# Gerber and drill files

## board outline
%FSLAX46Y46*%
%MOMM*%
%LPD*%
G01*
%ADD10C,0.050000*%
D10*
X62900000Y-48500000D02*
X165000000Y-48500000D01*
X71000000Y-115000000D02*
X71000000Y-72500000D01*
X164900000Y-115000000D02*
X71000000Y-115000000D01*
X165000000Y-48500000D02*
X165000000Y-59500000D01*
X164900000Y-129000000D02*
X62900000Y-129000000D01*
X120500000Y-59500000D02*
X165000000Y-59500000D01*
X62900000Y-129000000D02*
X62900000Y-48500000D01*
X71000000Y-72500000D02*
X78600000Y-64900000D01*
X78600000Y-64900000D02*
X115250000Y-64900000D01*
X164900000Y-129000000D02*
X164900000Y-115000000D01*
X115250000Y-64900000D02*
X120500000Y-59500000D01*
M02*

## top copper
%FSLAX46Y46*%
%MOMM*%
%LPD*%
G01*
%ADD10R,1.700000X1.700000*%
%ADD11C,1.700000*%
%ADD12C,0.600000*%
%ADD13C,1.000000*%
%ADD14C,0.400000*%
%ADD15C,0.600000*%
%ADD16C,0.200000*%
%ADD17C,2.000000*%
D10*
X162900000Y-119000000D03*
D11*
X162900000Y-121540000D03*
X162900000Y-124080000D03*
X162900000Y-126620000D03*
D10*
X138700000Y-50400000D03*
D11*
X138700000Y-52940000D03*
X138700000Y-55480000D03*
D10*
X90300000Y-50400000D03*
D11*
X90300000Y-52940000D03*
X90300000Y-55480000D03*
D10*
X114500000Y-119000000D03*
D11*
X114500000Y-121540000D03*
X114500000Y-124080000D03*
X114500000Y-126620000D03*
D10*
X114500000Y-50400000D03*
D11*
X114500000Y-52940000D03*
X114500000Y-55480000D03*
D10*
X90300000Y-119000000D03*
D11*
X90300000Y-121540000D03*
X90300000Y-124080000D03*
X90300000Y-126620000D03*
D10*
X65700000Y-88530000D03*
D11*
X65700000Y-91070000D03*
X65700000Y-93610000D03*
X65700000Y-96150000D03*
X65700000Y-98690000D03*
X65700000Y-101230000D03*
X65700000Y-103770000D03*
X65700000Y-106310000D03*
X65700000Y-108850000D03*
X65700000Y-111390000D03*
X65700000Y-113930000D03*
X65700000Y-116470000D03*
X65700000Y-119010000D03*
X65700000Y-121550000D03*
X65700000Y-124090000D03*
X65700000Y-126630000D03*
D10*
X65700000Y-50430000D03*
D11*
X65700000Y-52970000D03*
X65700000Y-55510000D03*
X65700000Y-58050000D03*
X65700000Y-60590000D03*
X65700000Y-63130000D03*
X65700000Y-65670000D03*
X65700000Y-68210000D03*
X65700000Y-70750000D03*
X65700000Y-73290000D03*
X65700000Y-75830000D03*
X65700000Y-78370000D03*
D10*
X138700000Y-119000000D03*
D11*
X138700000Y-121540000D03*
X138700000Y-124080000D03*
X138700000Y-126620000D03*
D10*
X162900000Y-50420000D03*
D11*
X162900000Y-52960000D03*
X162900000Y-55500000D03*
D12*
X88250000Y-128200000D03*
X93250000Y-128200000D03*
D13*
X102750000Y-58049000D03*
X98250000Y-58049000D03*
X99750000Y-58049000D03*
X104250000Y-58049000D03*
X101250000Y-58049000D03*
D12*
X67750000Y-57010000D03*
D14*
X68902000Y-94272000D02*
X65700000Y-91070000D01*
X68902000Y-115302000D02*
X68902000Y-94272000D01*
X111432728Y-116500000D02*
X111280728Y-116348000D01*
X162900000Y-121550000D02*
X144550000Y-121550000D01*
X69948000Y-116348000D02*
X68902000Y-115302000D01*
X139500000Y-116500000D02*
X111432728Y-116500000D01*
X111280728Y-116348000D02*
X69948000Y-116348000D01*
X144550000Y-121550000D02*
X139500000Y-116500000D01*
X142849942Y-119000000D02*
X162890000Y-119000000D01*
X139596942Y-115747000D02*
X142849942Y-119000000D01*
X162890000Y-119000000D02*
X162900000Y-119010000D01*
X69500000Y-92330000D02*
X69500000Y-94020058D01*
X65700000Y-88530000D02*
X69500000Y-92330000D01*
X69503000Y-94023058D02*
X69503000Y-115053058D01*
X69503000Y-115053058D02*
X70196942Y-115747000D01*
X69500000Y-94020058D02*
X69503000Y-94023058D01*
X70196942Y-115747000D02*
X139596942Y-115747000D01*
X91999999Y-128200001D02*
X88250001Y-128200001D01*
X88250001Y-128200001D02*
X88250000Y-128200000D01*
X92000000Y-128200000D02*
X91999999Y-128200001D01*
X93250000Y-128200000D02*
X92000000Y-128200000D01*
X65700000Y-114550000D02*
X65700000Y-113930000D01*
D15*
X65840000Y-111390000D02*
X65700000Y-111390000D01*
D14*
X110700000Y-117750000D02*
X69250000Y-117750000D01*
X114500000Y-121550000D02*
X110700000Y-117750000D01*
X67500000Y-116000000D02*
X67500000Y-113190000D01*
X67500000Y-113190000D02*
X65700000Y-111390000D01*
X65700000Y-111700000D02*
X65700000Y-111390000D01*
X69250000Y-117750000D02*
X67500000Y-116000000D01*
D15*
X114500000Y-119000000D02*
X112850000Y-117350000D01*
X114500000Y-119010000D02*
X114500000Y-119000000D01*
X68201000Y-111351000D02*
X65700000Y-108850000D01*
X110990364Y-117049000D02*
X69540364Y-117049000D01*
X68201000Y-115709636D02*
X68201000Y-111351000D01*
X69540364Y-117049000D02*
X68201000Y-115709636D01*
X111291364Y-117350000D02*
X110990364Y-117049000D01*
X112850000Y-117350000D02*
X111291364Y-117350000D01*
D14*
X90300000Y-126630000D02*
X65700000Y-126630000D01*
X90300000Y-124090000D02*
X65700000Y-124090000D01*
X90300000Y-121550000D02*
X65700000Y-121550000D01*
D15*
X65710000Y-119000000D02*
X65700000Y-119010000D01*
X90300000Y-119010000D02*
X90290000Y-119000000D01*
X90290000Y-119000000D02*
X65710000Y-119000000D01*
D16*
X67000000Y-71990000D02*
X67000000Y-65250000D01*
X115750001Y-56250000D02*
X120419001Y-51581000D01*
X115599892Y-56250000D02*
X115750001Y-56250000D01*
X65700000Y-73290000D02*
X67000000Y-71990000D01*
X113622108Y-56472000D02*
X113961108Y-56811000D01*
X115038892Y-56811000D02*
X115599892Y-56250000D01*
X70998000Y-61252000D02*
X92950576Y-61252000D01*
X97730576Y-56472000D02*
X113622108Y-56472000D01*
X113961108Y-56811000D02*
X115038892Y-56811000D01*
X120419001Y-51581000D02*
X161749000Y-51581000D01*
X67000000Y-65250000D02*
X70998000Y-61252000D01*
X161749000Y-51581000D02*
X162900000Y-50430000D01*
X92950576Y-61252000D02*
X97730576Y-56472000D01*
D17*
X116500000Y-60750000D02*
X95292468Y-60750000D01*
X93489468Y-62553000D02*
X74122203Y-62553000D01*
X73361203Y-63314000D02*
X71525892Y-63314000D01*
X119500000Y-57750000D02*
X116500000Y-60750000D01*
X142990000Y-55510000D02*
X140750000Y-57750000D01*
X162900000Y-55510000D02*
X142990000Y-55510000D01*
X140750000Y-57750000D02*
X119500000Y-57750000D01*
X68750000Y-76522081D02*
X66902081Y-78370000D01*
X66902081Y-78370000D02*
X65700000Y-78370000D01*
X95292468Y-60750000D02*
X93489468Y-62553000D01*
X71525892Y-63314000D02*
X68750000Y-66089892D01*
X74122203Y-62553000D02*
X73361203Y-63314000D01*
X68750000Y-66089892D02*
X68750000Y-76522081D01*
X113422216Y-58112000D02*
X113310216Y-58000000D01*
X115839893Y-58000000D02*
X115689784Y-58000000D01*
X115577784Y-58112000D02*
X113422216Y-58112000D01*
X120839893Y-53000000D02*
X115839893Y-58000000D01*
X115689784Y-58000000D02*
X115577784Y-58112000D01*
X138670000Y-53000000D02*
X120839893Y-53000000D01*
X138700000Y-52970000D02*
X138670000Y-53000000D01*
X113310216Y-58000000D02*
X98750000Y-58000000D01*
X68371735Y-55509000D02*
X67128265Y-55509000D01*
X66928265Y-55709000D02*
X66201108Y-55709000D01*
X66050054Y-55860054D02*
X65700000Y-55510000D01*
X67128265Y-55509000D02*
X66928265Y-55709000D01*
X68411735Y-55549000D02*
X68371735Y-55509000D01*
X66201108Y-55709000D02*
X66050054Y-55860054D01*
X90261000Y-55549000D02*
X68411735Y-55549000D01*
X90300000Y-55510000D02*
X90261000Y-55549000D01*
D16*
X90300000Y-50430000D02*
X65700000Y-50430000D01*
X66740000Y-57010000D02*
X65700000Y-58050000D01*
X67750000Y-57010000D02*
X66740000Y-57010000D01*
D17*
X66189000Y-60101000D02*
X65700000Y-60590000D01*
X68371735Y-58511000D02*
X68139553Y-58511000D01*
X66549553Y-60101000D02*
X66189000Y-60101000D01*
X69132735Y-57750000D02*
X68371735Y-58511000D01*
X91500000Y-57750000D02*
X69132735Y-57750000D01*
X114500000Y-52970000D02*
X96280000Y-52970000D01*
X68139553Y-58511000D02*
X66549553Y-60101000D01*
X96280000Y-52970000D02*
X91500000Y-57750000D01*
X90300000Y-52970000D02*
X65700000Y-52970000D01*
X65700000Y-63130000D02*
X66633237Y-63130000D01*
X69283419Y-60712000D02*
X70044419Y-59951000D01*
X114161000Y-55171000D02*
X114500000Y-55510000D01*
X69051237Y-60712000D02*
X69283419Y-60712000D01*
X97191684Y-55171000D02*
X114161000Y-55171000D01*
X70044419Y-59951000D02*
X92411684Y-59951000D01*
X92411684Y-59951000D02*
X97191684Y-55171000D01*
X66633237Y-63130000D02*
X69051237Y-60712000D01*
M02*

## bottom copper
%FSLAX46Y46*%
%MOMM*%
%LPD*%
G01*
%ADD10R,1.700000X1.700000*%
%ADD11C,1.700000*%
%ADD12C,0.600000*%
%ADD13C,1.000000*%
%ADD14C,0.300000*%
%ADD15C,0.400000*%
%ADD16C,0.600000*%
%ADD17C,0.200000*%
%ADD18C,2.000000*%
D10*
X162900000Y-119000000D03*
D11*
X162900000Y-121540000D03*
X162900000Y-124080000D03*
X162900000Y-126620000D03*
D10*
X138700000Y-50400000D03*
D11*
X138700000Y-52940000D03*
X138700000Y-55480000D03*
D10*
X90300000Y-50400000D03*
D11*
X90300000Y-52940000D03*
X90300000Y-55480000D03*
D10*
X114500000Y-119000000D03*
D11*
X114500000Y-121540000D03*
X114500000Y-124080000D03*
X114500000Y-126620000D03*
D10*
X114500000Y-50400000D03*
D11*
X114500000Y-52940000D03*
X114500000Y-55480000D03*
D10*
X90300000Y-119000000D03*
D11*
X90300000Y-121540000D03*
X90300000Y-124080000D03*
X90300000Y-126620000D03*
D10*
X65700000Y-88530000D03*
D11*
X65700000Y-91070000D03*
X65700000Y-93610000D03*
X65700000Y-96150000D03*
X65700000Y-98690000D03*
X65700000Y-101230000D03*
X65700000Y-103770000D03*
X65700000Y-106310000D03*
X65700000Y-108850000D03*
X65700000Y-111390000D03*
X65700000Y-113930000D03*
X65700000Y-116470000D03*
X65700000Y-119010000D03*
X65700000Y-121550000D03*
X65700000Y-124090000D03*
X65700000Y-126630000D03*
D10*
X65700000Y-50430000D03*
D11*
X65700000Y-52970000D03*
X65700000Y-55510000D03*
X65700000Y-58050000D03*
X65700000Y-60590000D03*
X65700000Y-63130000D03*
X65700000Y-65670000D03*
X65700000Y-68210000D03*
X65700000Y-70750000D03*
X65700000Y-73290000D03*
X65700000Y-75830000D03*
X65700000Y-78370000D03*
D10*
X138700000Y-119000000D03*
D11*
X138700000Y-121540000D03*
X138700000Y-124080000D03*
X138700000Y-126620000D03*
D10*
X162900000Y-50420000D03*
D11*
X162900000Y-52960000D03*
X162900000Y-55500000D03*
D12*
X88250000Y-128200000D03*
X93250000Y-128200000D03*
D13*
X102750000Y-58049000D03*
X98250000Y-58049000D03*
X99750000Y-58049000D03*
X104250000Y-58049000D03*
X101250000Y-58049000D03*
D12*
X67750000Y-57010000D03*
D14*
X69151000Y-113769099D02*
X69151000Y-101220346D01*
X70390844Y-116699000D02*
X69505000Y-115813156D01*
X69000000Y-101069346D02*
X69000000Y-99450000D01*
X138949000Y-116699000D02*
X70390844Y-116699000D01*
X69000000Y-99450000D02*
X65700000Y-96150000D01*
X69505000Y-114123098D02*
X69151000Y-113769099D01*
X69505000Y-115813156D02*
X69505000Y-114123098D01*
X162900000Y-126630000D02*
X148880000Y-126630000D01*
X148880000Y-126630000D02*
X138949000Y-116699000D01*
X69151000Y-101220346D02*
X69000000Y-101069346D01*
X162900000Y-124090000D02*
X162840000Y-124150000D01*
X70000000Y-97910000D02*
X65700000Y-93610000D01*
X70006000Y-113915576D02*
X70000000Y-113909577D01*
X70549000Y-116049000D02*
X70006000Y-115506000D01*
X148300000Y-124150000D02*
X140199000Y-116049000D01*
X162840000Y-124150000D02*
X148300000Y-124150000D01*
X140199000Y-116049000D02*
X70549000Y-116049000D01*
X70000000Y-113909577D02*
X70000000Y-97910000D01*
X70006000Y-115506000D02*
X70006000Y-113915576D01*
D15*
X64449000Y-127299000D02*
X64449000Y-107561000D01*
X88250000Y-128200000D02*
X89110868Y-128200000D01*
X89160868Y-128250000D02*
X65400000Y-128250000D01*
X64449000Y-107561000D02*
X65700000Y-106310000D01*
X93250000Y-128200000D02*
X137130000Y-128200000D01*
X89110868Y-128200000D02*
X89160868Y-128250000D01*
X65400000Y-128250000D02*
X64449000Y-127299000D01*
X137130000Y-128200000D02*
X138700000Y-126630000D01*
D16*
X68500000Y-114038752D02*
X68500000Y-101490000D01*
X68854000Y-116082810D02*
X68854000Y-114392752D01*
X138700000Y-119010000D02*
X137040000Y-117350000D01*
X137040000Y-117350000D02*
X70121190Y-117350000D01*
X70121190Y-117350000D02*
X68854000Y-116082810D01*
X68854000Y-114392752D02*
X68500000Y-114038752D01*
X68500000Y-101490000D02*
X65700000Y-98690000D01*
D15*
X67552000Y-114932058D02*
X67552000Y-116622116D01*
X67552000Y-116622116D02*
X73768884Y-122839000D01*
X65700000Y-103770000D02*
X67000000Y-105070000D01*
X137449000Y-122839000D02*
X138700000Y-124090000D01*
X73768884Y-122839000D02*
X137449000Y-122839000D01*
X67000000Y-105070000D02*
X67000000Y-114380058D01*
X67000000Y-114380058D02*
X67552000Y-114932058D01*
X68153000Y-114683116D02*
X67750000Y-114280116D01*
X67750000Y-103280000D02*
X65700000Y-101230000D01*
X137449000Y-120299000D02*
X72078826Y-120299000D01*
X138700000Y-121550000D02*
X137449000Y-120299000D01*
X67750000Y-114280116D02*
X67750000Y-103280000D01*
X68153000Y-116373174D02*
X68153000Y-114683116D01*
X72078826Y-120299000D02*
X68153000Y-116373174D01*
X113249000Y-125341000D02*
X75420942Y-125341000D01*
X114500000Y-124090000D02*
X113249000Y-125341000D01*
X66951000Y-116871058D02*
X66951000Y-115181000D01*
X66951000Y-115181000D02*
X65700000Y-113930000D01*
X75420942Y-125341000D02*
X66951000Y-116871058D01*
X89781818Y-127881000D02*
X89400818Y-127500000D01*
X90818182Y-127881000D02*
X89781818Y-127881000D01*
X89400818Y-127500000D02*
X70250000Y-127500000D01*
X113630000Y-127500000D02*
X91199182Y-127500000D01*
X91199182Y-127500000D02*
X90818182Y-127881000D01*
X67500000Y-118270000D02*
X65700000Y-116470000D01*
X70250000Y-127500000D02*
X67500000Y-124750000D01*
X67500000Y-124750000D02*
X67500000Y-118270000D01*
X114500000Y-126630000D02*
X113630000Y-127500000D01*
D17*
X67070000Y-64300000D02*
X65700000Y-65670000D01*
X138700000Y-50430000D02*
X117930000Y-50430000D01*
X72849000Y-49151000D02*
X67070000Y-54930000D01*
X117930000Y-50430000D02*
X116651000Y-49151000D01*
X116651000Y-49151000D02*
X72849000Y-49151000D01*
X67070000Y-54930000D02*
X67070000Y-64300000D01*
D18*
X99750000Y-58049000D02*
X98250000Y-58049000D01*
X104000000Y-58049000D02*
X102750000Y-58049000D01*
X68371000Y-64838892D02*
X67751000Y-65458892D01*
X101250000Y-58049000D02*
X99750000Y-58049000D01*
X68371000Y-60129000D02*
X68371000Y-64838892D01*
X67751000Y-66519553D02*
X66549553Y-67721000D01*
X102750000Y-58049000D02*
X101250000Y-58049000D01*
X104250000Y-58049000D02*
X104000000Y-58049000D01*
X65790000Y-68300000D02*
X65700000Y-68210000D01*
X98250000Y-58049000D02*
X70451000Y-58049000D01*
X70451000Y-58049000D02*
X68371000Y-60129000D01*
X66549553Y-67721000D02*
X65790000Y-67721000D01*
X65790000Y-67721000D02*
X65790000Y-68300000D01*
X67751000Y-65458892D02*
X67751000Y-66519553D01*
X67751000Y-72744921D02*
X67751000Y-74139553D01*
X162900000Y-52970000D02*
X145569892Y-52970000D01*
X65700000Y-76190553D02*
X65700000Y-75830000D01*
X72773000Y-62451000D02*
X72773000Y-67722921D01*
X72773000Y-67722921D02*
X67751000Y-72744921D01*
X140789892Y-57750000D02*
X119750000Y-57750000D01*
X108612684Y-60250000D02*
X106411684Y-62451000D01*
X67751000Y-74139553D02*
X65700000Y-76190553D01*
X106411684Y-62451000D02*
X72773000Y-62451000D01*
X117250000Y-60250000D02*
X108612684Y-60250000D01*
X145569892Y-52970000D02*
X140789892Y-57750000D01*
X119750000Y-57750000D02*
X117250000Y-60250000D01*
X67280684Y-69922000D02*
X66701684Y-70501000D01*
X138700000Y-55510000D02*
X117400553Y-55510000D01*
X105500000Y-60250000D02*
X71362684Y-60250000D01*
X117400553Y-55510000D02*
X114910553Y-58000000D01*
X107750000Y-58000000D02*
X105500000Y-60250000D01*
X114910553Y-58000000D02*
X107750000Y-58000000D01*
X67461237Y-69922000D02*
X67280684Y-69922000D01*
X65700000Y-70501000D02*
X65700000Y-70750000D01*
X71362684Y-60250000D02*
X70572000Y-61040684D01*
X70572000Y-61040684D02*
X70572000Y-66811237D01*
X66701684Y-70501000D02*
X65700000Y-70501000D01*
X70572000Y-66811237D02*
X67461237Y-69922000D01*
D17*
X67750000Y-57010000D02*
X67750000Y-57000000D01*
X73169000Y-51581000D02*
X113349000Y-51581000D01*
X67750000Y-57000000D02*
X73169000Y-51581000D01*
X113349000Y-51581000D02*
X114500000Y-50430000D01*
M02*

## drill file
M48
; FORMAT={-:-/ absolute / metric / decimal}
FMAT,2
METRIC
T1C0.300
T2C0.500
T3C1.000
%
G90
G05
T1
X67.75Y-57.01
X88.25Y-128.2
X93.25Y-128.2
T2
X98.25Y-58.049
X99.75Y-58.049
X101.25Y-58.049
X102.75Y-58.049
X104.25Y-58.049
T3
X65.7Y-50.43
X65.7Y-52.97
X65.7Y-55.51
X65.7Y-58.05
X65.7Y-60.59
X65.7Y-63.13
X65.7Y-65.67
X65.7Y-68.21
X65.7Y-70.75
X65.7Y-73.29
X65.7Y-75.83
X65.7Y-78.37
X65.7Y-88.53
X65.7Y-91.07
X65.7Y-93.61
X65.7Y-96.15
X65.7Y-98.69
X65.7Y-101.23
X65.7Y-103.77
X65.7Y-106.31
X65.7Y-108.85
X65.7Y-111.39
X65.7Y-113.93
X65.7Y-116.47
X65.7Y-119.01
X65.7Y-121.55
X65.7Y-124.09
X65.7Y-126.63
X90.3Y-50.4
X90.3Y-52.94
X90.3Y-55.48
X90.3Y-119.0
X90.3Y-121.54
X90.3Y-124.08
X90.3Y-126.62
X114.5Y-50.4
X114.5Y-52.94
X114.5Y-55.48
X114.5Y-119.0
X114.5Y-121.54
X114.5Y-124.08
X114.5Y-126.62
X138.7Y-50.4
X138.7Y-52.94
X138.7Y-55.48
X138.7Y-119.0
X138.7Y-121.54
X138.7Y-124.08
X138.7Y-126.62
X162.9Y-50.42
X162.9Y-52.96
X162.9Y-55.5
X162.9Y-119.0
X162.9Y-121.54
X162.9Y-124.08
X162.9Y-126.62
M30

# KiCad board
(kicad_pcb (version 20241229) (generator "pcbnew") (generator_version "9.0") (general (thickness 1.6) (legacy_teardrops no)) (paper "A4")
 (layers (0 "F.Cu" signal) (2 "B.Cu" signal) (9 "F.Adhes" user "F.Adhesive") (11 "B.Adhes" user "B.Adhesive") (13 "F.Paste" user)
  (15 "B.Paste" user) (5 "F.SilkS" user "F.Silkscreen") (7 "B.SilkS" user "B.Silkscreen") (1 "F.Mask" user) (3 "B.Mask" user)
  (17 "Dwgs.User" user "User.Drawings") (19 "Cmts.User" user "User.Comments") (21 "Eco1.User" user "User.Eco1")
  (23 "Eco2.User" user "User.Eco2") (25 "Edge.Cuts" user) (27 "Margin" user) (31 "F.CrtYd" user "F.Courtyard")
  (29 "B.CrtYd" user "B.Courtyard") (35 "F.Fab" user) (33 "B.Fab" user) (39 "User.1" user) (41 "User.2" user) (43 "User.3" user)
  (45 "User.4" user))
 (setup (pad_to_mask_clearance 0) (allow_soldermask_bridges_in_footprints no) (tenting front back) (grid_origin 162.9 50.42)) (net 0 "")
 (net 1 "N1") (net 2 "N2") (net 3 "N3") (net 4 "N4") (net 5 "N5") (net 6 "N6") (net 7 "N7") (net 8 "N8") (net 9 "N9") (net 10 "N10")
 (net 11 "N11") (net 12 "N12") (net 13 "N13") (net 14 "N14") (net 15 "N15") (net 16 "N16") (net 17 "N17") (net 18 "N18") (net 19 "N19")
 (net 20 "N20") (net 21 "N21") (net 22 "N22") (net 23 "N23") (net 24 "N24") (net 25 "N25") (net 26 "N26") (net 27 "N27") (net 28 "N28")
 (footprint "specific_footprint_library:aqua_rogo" (layer "F.Cu") (at 72 64 -90)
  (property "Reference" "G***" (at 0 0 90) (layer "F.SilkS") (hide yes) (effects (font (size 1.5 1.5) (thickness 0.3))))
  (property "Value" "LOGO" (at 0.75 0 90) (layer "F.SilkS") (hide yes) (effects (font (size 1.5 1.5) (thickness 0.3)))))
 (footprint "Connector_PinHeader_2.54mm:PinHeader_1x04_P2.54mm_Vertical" (layer "B.Cu") (at 162.9 119 180)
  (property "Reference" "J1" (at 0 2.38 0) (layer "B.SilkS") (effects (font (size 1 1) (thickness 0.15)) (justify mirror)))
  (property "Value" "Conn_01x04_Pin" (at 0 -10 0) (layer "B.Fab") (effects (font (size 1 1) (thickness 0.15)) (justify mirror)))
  (pad "1" thru_hole rect (at 0 0 180) (size 1.7 1.7) (drill 1) (layers "*.Cu" "*.Mask") (remove_unused_layers no) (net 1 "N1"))
  (pad "2" thru_hole circle (at 0 -2.54 180) (size 1.7 1.7) (drill 1) (layers "*.Cu" "*.Mask") (remove_unused_layers no) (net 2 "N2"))
  (pad "3" thru_hole circle (at 0 -5.08 180) (size 1.7 1.7) (drill 1) (layers "*.Cu" "*.Mask") (remove_unused_layers no) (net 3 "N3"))
  (pad "4" thru_hole circle (at 0 -7.62 180) (size 1.7 1.7) (drill 1) (layers "*.Cu" "*.Mask") (remove_unused_layers no) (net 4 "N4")))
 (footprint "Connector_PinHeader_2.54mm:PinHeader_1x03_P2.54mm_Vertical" (layer "B.Cu") (at 138.7 50.4 180)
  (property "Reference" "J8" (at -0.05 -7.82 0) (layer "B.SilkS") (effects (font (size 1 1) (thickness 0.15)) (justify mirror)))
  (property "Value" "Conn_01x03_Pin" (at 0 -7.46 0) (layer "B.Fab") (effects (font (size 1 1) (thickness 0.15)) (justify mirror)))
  (pad "1" thru_hole rect (at 0 0 180) (size 1.7 1.7) (drill 1) (layers "*.Cu" "*.Mask") (remove_unused_layers no) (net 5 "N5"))
  (pad "2" thru_hole circle (at 0 -2.54 180) (size 1.7 1.7) (drill 1) (layers "*.Cu" "*.Mask") (remove_unused_layers no) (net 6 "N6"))
  (pad "3" thru_hole circle (at 0 -5.08 180) (size 1.7 1.7) (drill 1) (layers "*.Cu" "*.Mask") (remove_unused_layers no) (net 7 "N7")))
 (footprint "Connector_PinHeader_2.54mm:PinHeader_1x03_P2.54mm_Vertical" (layer "B.Cu") (at 90.3 50.4 180)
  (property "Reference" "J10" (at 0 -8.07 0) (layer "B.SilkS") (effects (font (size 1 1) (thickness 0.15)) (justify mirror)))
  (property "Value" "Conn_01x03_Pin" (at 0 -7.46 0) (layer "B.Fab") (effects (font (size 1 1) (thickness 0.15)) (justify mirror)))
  (pad "1" thru_hole rect (at 0 0 180) (size 1.7 1.7) (drill 1) (layers "*.Cu" "*.Mask") (remove_unused_layers no) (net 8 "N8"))
  (pad "2" thru_hole circle (at 0 -2.54 180) (size 1.7 1.7) (drill 1) (layers "*.Cu" "*.Mask") (remove_unused_layers no) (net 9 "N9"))
  (pad "3" thru_hole circle (at 0 -5.08 180) (size 1.7 1.7) (drill 1) (layers "*.Cu" "*.Mask") (remove_unused_layers no) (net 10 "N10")))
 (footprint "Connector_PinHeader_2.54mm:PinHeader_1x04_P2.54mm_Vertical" (layer "B.Cu") (at 114.5 119 180)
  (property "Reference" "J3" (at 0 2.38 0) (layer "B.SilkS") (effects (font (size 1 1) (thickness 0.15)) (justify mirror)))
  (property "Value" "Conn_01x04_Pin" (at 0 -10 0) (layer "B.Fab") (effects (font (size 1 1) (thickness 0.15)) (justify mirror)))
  (pad "1" thru_hole rect (at 0 0 180) (size 1.7 1.7) (drill 1) (layers "*.Cu" "*.Mask") (remove_unused_layers no) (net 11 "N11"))
  (pad "2" thru_hole circle (at 0 -2.54 180) (size 1.7 1.7) (drill 1) (layers "*.Cu" "*.Mask") (remove_unused_layers no) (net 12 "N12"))
  (pad "3" thru_hole circle (at 0 -5.08 180) (size 1.7 1.7) (drill 1) (layers "*.Cu" "*.Mask") (remove_unused_layers no) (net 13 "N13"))
  (pad "4" thru_hole circle (at 0 -7.62 180) (size 1.7 1.7) (drill 1) (layers "*.Cu" "*.Mask") (remove_unused_layers no) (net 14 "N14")))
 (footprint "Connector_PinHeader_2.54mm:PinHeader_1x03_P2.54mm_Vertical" (layer "B.Cu") (at 114.5 50.4 180)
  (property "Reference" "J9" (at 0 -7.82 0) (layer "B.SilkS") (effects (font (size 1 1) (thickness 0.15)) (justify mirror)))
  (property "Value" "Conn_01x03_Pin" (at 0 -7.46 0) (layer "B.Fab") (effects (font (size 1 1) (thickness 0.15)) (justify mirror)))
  (pad "1" thru_hole rect (at 0 0 180) (size 1.7 1.7) (drill 1) (layers "*.Cu" "*.Mask") (remove_unused_layers no) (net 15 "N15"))
  (pad "2" thru_hole circle (at 0 -2.54 180) (size 1.7 1.7) (drill 1) (layers "*.Cu" "*.Mask") (remove_unused_layers no) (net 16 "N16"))
  (pad "3" thru_hole circle (at 0 -5.08 180) (size 1.7 1.7) (drill 1) (layers "*.Cu" "*.Mask") (remove_unused_layers no) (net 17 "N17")))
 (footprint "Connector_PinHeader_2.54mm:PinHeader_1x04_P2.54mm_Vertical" (layer "B.Cu") (at 90.3 119 180)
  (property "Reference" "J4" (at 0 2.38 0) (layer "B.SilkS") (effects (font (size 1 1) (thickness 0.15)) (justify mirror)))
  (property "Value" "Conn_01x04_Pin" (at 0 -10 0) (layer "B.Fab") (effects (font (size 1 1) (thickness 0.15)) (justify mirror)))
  (pad "1" thru_hole rect (at 0 0 180) (size 1.7 1.7) (drill 1) (layers "*.Cu" "*.Mask") (remove_unused_layers no) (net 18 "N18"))
  (pad "2" thru_hole circle (at 0 -2.54 180) (size 1.7 1.7) (drill 1) (layers "*.Cu" "*.Mask") (remove_unused_layers no) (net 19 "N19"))
  (pad "3" thru_hole circle (at 0 -5.08 180) (size 1.7 1.7) (drill 1) (layers "*.Cu" "*.Mask") (remove_unused_layers no) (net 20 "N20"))
  (pad "4" thru_hole circle (at 0 -7.62 180) (size 1.7 1.7) (drill 1) (layers "*.Cu" "*.Mask") (remove_unused_layers no) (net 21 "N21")))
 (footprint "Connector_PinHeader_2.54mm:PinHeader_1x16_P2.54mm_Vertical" (layer "B.Cu") (at 65.7 88.53 180)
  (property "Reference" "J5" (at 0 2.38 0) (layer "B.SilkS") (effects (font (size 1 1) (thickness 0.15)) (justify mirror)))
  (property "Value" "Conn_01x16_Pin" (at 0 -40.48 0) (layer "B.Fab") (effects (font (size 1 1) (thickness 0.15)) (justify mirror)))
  (pad "1" thru_hole rect (at 0 0 180) (size 1.7 1.7) (drill 1) (layers "*.Cu" "*.Mask") (remove_unused_layers no) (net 1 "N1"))
  (pad "2" thru_hole circle (at 0 -2.54 180) (size 1.7 1.7) (drill 1) (layers "*.Cu" "*.Mask") (remove_unused_layers no) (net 2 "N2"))
  (pad "3" thru_hole circle (at 0 -5.08 180) (size 1.7 1.7) (drill 1) (layers "*.Cu" "*.Mask") (remove_unused_layers no) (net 3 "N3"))
  (pad "4" thru_hole circle (at 0 -7.62 180) (size 1.7 1.7) (drill 1) (layers "*.Cu" "*.Mask") (remove_unused_layers no) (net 4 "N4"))
  (pad "5" thru_hole circle (at 0 -10.16 180) (size 1.7 1.7) (drill 1) (layers "*.Cu" "*.Mask") (remove_unused_layers no) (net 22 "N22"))
  (pad "6" thru_hole circle (at 0 -12.7 180) (size 1.7 1.7) (drill 1) (layers "*.Cu" "*.Mask") (remove_unused_layers no) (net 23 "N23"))
  (pad "7" thru_hole circle (at 0 -15.24 180) (size 1.7 1.7) (drill 1) (layers "*.Cu" "*.Mask") (remove_unused_layers no) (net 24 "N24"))
  (pad "8" thru_hole circle (at 0 -17.78 180) (size 1.7 1.7) (drill 1) (layers "*.Cu" "*.Mask") (remove_unused_layers no) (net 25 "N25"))
  (pad "9" thru_hole circle (at 0 -20.32 180) (size 1.7 1.7) (drill 1) (layers "*.Cu" "*.Mask") (remove_unused_layers no) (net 11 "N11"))
  (pad "10" thru_hole circle (at 0 -22.86 180) (size 1.7 1.7) (drill 1) (layers "*.Cu" "*.Mask") (remove_unused_layers no) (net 12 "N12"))
  (pad "11" thru_hole circle (at 0 -25.4 180) (size 1.7 1.7) (drill 1) (layers "*.Cu" "*.Mask") (remove_unused_layers no) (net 13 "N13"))
  (pad "12" thru_hole circle (at 0 -27.94 180) (size 1.7 1.7) (drill 1) (layers "*.Cu" "*.Mask") (remove_unused_layers no) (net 14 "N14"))
  (pad "13" thru_hole circle (at 0 -30.48 180) (size 1.7 1.7) (drill 1) (layers "*.Cu" "*.Mask") (remove_unused_layers no) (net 18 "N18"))
  (pad "14" thru_hole circle (at 0 -33.02 180) (size 1.7 1.7) (drill 1) (layers "*.Cu" "*.Mask") (remove_unused_layers no) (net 19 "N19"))
  (pad "15" thru_hole circle (at 0 -35.56 180) (size 1.7 1.7) (drill 1) (layers "*.Cu" "*.Mask") (remove_unused_layers no) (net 20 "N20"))
  (pad "16" thru_hole circle (at 0 -38.1 180) (size 1.7 1.7) (drill 1) (layers "*.Cu" "*.Mask") (remove_unused_layers no) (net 21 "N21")))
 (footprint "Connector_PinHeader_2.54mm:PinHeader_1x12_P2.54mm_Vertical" (layer "B.Cu") (at 65.7 50.43 180)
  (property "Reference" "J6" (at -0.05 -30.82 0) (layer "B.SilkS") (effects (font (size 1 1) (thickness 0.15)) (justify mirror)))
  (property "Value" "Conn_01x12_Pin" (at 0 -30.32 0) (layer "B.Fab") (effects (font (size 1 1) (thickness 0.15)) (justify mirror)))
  (pad "1" thru_hole rect (at 0 0 180) (size 1.7 1.7) (drill 1) (layers "*.Cu" "*.Mask") (remove_unused_layers no) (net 8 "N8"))
  (pad "2" thru_hole circle (at 0 -2.54 180) (size 1.7 1.7) (drill 1) (layers "*.Cu" "*.Mask") (remove_unused_layers no) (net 9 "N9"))
  (pad "3" thru_hole circle (at 0 -5.08 180) (size 1.7 1.7) (drill 1) (layers "*.Cu" "*.Mask") (remove_unused_layers no) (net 10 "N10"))
  (pad "4" thru_hole circle (at 0 -7.62 180) (size 1.7 1.7) (drill 1) (layers "*.Cu" "*.Mask") (remove_unused_layers no) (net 15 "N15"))
  (pad "5" thru_hole circle (at 0 -10.16 180) (size 1.7 1.7) (drill 1) (layers "*.Cu" "*.Mask") (remove_unused_layers no) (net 16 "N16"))
  (pad "6" thru_hole circle (at 0 -12.7 180) (size 1.7 1.7) (drill 1) (layers "*.Cu" "*.Mask") (remove_unused_layers no) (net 17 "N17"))
  (pad "7" thru_hole circle (at 0 -15.24 180) (size 1.7 1.7) (drill 1) (layers "*.Cu" "*.Mask") (remove_unused_layers no) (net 5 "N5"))
  (pad "8" thru_hole circle (at 0 -17.78 180) (size 1.7 1.7) (drill 1) (layers "*.Cu" "*.Mask") (remove_unused_layers no) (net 6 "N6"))
  (pad "9" thru_hole circle (at 0 -20.32 180) (size 1.7 1.7) (drill 1) (layers "*.Cu" "*.Mask") (remove_unused_layers no) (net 7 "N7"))
  (pad "10" thru_hole circle (at 0 -22.86 180) (size 1.7 1.7) (drill 1) (layers "*.Cu" "*.Mask") (remove_unused_layers no) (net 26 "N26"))
  (pad "11" thru_hole circle (at 0 -25.4 180) (size 1.7 1.7) (drill 1) (layers "*.Cu" "*.Mask") (remove_unused_layers no) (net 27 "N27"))
  (pad "12" thru_hole circle (at 0 -27.94 180) (size 1.7 1.7) (drill 1) (layers "*.Cu" "*.Mask") (remove_unused_layers no) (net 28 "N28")))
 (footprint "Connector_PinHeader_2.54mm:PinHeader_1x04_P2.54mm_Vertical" (layer "B.Cu") (at 138.7 119 180)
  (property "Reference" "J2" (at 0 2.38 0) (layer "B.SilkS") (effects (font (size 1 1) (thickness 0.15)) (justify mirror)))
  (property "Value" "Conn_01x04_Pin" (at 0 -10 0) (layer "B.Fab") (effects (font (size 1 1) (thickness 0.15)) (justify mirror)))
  (pad "1" thru_hole rect (at 0 0 180) (size 1.7 1.7) (drill 1) (layers "*.Cu" "*.Mask") (remove_unused_layers no) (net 22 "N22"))
  (pad "2" thru_hole circle (at 0 -2.54 180) (size 1.7 1.7) (drill 1) (layers "*.Cu" "*.Mask") (remove_unused_layers no) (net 23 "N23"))
  (pad "3" thru_hole circle (at 0 -5.08 180) (size 1.7 1.7) (drill 1) (layers "*.Cu" "*.Mask") (remove_unused_layers no) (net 24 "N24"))
  (pad "4" thru_hole circle (at 0 -7.62 180) (size 1.7 1.7) (drill 1) (layers "*.Cu" "*.Mask") (remove_unused_layers no) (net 25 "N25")))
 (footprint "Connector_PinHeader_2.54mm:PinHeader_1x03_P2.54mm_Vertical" (layer "B.Cu") (at 162.9 50.42 180)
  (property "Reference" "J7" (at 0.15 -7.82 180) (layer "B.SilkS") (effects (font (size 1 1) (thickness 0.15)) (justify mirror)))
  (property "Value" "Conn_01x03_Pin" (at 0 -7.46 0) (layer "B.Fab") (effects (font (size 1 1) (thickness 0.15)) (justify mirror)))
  (pad "1" thru_hole rect (at 0 0 180) (size 1.7 1.7) (drill 1) (layers "*.Cu" "*.Mask") (remove_unused_layers no) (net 26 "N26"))
  (pad "2" thru_hole circle (at 0 -2.54 180) (size 1.7 1.7) (drill 1) (layers "*.Cu" "*.Mask") (remove_unused_layers no) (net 27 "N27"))
  (pad "3" thru_hole circle (at 0 -5.08 180) (size 1.7 1.7) (drill 1) (layers "*.Cu" "*.Mask") (remove_unused_layers no) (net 28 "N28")))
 (gr_line (start 62.9 48.5) (end 165 48.5) (stroke (width 0.05) (type default)) (layer "Edge.Cuts"))
 (gr_line (start 71 115) (end 71 72.5) (stroke (width 0.05) (type default)) (layer "Edge.Cuts"))
 (gr_line (start 164.9 115) (end 71 115) (stroke (width 0.05) (type default)) (layer "Edge.Cuts"))
 (gr_line (start 165 48.5) (end 165 59.5) (stroke (width 0.05) (type default)) (layer "Edge.Cuts"))
 (gr_line (start 164.9 129) (end 62.9 129) (stroke (width 0.05) (type solid)) (layer "Edge.Cuts"))
 (gr_line (start 120.5 59.5) (end 165 59.5) (stroke (width 0.05) (type default)) (layer "Edge.Cuts"))
 (gr_line (start 62.9 129) (end 62.9 48.5) (stroke (width 0.05) (type default)) (layer "Edge.Cuts"))
 (gr_line (start 71 72.5) (end 78.6 64.9) (stroke (width 0.05) (type default)) (layer "Edge.Cuts"))
 (gr_line (start 78.6 64.9) (end 115.25 64.9) (stroke (width 0.05) (type default)) (layer "Edge.Cuts"))
 (gr_line (start 164.9 129) (end 164.9 115) (stroke (width 0.05) (type default)) (layer "Edge.Cuts"))
 (gr_line (start 115.25 64.9) (end 120.5 59.5) (stroke (width 0.05) (type default)) (layer "Edge.Cuts"))
 (segment (start 68.902 94.272) (end 65.7 91.07) (width 0.4) (layer "F.Cu") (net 2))
 (segment (start 68.902 115.302) (end 68.902 94.272) (width 0.4) (layer "F.Cu") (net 2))
 (segment (start 111.432728 116.5) (end 111.280728 116.348) (width 0.4) (layer "F.Cu") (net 2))
 (segment (start 162.9 121.55) (end 144.55 121.55) (width 0.4) (layer "F.Cu") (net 2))
 (segment (start 69.948 116.348) (end 68.902 115.302) (width 0.4) (layer "F.Cu") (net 2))
 (segment (start 139.5 116.5) (end 111.432728 116.5) (width 0.4) (layer "F.Cu") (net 2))
 (segment (start 111.280728 116.348) (end 69.948 116.348) (width 0.4) (layer "F.Cu") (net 2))
 (segment (start 144.55 121.55) (end 139.5 116.5) (width 0.4) (layer "F.Cu") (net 2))
 (segment (start 69.151 113.769099) (end 69.151 101.220346) (width 0.3) (layer "B.Cu") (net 4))
 (segment (start 70.390844 116.699) (end 69.505 115.813156) (width 0.3) (layer "B.Cu") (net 4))
 (segment (start 69 101.069346) (end 69 99.45) (width 0.3) (layer "B.Cu") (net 4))
 (segment (start 138.949 116.699) (end 70.390844 116.699) (width 0.3) (layer "B.Cu") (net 4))
 (segment (start 69 99.45) (end 65.7 96.15) (width 0.3) (layer "B.Cu") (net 4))
 (segment (start 69.505 114.123098) (end 69.151 113.769099) (width 0.3) (layer "B.Cu") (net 4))
 (segment (start 69.505 115.813156) (end 69.505 114.123098) (width 0.3) (layer "B.Cu") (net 4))
 (segment (start 162.9 126.63) (end 148.88 126.63) (width 0.3) (layer "B.Cu") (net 4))
 (segment (start 148.88 126.63) (end 138.949 116.699) (width 0.3) (layer "B.Cu") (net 4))
 (segment (start 69.151 101.220346) (end 69 101.069346) (width 0.3) (layer "B.Cu") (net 4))
 (segment (start 142.849942 119) (end 162.89 119) (width 0.4) (layer "F.Cu") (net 1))
 (segment (start 139.596942 115.747) (end 142.849942 119) (width 0.4) (layer "F.Cu") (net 1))
 (segment (start 162.89 119) (end 162.9 119.01) (width 0.4) (layer "F.Cu") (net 1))
 (segment (start 69.5 92.33) (end 69.5 94.020058) (width 0.4) (layer "F.Cu") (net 1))
 (segment (start 65.7 88.53) (end 69.5 92.33) (width 0.4) (layer "F.Cu") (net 1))
 (segment (start 69.503 94.023058) (end 69.503 115.053058) (width 0.4) (layer "F.Cu") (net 1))
 (segment (start 69.503 115.053058) (end 70.196942 115.747) (width 0.4) (layer "F.Cu") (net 1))
 (segment (start 69.5 94.020058) (end 69.503 94.023058) (width 0.4) (layer "F.Cu") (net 1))
 (segment (start 70.196942 115.747) (end 139.596942 115.747) (width 0.4) (layer "F.Cu") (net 1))
 (segment (start 162.9 124.09) (end 162.84 124.15) (width 0.3) (layer "B.Cu") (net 3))
 (segment (start 70 97.91) (end 65.7 93.61) (width 0.3) (layer "B.Cu") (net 3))
 (segment (start 70.006 113.915576) (end 70 113.909577) (width 0.3) (layer "B.Cu") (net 3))
 (segment (start 70.549 116.049) (end 70.006 115.506) (width 0.3) (layer "B.Cu") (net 3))
 (segment (start 148.3 124.15) (end 140.199 116.049) (width 0.3) (layer "B.Cu") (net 3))
 (segment (start 162.84 124.15) (end 148.3 124.15) (width 0.3) (layer "B.Cu") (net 3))
 (segment (start 140.199 116.049) (end 70.549 116.049) (width 0.3) (layer "B.Cu") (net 3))
 (segment (start 70 113.909577) (end 70 97.91) (width 0.3) (layer "B.Cu") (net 3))
 (segment (start 70.006 115.506) (end 70.006 113.915576) (width 0.3) (layer "B.Cu") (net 3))
 (segment (start 91.999999 128.200001) (end 88.250001 128.200001) (width 0.4) (layer "F.Cu") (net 25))
 (segment (start 88.250001 128.200001) (end 88.25 128.2) (width 0.4) (layer "F.Cu") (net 25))
 (segment (start 92 128.2) (end 91.999999 128.200001) (width 0.4) (layer "F.Cu") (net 25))
 (segment (start 93.25 128.2) (end 92 128.2) (width 0.4) (layer "F.Cu") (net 25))
 (via (at 88.25 128.2) (size 0.6) (drill 0.3) (layers "F.Cu" "B.Cu") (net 25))
 (via (at 93.25 128.2) (size 0.6) (drill 0.3) (layers "F.Cu" "B.Cu") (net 25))
 (segment (start 64.449 127.299) (end 64.449 107.561) (width 0.4) (layer "B.Cu") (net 25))
 (segment (start 88.25 128.2) (end 89.110868 128.2) (width 0.4) (layer "B.Cu") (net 25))
 (segment (start 89.160868 128.25) (end 65.4 128.25) (width 0.4) (layer "B.Cu") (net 25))
 (segment (start 64.449 107.561) (end 65.7 106.31) (width 0.4) (layer "B.Cu") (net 25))
 (segment (start 93.25 128.2) (end 137.13 128.2) (width 0.4) (layer "B.Cu") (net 25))
 (segment (start 89.110868 128.2) (end 89.160868 128.25) (width 0.4) (layer "B.Cu") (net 25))
 (segment (start 65.4 128.25) (end 64.449 127.299) (width 0.4) (layer "B.Cu") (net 25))
 (segment (start 137.13 128.2) (end 138.7 126.63) (width 0.4) (layer "B.Cu") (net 25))
 (segment (start 68.5 114.038752) (end 68.5 101.49) (width 0.6) (layer "B.Cu") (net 22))
 (segment (start 68.854 116.08281) (end 68.854 114.392752) (width 0.6) (layer "B.Cu") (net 22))
 (segment (start 138.7 119.01) (end 137.04 117.35) (width 0.6) (layer "B.Cu") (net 22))
 (segment (start 137.04 117.35) (end 70.12119 117.35) (width 0.6) (layer "B.Cu") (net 22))
 (segment (start 70.12119 117.35) (end 68.854 116.08281) (width 0.6) (layer "B.Cu") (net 22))
 (segment (start 68.854 114.392752) (end 68.5 114.038752) (width 0.6) (layer "B.Cu") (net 22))
 (segment (start 68.5 101.49) (end 65.7 98.69) (width 0.6) (layer "B.Cu") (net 22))
 (segment (start 67.552 114.932058) (end 67.552 116.622116) (width 0.4) (layer "B.Cu") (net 24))
 (segment (start 67.552 116.622116) (end 73.768884 122.839) (width 0.4) (layer "B.Cu") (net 24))
 (segment (start 65.7 103.77) (end 67 105.07) (width 0.4) (layer "B.Cu") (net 24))
 (segment (start 137.449 122.839) (end 138.7 124.09) (width 0.4) (layer "B.Cu") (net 24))
 (segment (start 73.768884 122.839) (end 137.449 122.839) (width 0.4) (layer "B.Cu") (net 24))
 (segment (start 67 105.07) (end 67 114.380058) (width 0.4) (layer "B.Cu") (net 24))
 (segment (start 67 114.380058) (end 67.552 114.932058) (width 0.4) (layer "B.Cu") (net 24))
 (segment (start 68.153 114.683116) (end 67.75 114.280116) (width 0.4) (layer "B.Cu") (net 23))
 (segment (start 67.75 103.28) (end 65.7 101.23) (width 0.4) (layer "B.Cu") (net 23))
 (segment (start 137.449 120.299) (end 72.078826 120.299) (width 0.4) (layer "B.Cu") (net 23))
 (segment (start 138.7 121.55) (end 137.449 120.299) (width 0.4) (layer "B.Cu") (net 23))
 (segment (start 67.75 114.280116) (end 67.75 103.28) (width 0.4) (layer "B.Cu") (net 23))
 (segment (start 68.153 116.373174) (end 68.153 114.683116) (width 0.4) (layer "B.Cu") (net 23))
 (segment (start 72.078826 120.299) (end 68.153 116.373174) (width 0.4) (layer "B.Cu") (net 23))
 (segment (start 65.7 114.55) (end 65.7 113.93) (width 0.4) (layer "F.Cu") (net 13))
 (segment (start 113.249 125.341) (end 75.420942 125.341) (width 0.4) (layer "B.Cu") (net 13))
 (segment (start 114.5 124.09) (end 113.249 125.341) (width 0.4) (layer "B.Cu") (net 13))
 (segment (start 66.951 116.871058) (end 66.951 115.181) (width 0.4) (layer "B.Cu") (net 13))
 (segment (start 66.951 115.181) (end 65.7 113.93) (width 0.4) (layer "B.Cu") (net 13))
 (segment (start 75.420942 125.341) (end 66.951 116.871058) (width 0.4) (layer "B.Cu") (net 13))
 (segment (start 65.84 111.39) (end 65.7 111.39) (width 0.6) (layer "F.Cu") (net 12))
 (segment (start 110.7 117.75) (end 69.25 117.75) (width 0.4) (layer "F.Cu") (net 12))
 (segment (start 114.5 121.55) (end 110.7 117.75) (width 0.4) (layer "F.Cu") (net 12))
 (segment (start 67.5 116) (end 67.5 113.19) (width 0.4) (layer "F.Cu") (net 12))
 (segment (start 67.5 113.19) (end 65.7 111.39) (width 0.4) (layer "F.Cu") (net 12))
 (segment (start 65.7 111.7) (end 65.7 111.39) (width 0.4) (layer "F.Cu") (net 12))
 (segment (start 69.25 117.75) (end 67.5 116) (width 0.4) (layer "F.Cu") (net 12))
 (segment (start 114.5 119) (end 112.85 117.35) (width 0.6) (layer "F.Cu") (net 11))
 (segment (start 114.5 119.01) (end 114.5 119) (width 0.6) (layer "F.Cu") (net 11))
 (segment (start 68.201 111.351) (end 65.7 108.85) (width 0.6) (layer "F.Cu") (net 11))
 (segment (start 110.990364 117.049) (end 69.540364 117.049) (width 0.6) (layer "F.Cu") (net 11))
 (segment (start 68.201 115.709636) (end 68.201 111.351) (width 0.6) (layer "F.Cu") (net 11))
 (segment (start 69.540364 117.049) (end 68.201 115.709636) (width 0.6) (layer "F.Cu") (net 11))
 (segment (start 111.291364 117.35) (end 110.990364 117.049) (width 0.6) (layer "F.Cu") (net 11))
 (segment (start 112.85 117.35) (end 111.291364 117.35) (width 0.6) (layer "F.Cu") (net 11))
 (segment (start 89.781818 127.881) (end 89.400818 127.5) (width 0.4) (layer "B.Cu") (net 14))
 (segment (start 90.818182 127.881) (end 89.781818 127.881) (width 0.4) (layer "B.Cu") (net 14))
 (segment (start 89.400818 127.5) (end 70.25 127.5) (width 0.4) (layer "B.Cu") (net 14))
 (segment (start 113.63 127.5) (end 91.199182 127.5) (width 0.4) (layer "B.Cu") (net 14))
 (segment (start 91.199182 127.5) (end 90.818182 127.881) (width 0.4) (layer "B.Cu") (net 14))
 (segment (start 67.5 118.27) (end 65.7 116.47) (width 0.4) (layer "B.Cu") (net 14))
 (segment (start 70.25 127.5) (end 67.5 124.75) (width 0.4) (layer "B.Cu") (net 14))
 (segment (start 67.5 124.75) (end 67.5 118.27) (width 0.4) (layer "B.Cu") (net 14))
 (segment (start 114.5 126.63) (end 113.63 127.5) (width 0.4) (layer "B.Cu") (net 14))
 (segment (start 90.3 126.63) (end 65.7 126.63) (width 0.4) (layer "F.Cu") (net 21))
 (segment (start 90.3 124.09) (end 65.7 124.09) (width 0.4) (layer "F.Cu") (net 20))
 (segment (start 90.3 121.55) (end 65.7 121.55) (width 0.4) (layer "F.Cu") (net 19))
 (segment (start 65.71 119) (end 65.7 119.01) (width 0.6) (layer "F.Cu") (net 18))
 (segment (start 90.3 119.01) (end 90.29 119) (width 0.6) (layer "F.Cu") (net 18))
 (segment (start 90.29 119) (end 65.71 119) (width 0.6) (layer "F.Cu") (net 18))
 (segment (start 67.07 64.3) (end 65.7 65.67) (width 0.2) (layer "B.Cu") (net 5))
 (segment (start 138.7 50.43) (end 117.93 50.43) (width 0.2) (layer "B.Cu") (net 5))
 (segment (start 72.849 49.151) (end 67.07 54.93) (width 0.2) (layer "B.Cu") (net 5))
 (segment (start 117.93 50.43) (end 116.651 49.151) (width 0.2) (layer "B.Cu") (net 5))
 (segment (start 116.651 49.151) (end 72.849 49.151) (width 0.2) (layer "B.Cu") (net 5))
 (segment (start 67.07 54.93) (end 67.07 64.3) (width 0.2) (layer "B.Cu") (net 5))
 (segment (start 67 71.99) (end 67 65.25) (width 0.2) (layer "F.Cu") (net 26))
 (segment (start 115.750001 56.25) (end 120.419001 51.581) (width 0.2) (layer "F.Cu") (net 26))
 (segment (start 115.599892 56.25) (end 115.750001 56.25) (width 0.2) (layer "F.Cu") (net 26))
 (segment (start 65.7 73.29) (end 67 71.99) (width 0.2) (layer "F.Cu") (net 26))
 (segment (start 113.622108 56.472) (end 113.961108 56.811) (width 0.2) (layer "F.Cu") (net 26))
 (segment (start 115.038892 56.811) (end 115.599892 56.25) (width 0.2) (layer "F.Cu") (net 26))
 (segment (start 70.998 61.252) (end 92.950576 61.252) (width 0.2) (layer "F.Cu") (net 26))
 (segment (start 97.730576 56.472) (end 113.622108 56.472) (width 0.2) (layer "F.Cu") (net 26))
 (segment (start 113.961108 56.811) (end 115.038892 56.811) (width 0.2) (layer "F.Cu") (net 26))
 (segment (start 120.419001 51.581) (end 161.749 51.581) (width 0.2) (layer "F.Cu") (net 26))
 (segment (start 67 65.25) (end 70.998 61.252) (width 0.2) (layer "F.Cu") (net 26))
 (segment (start 161.749 51.581) (end 162.9 50.43) (width 0.2) (layer "F.Cu") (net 26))
 (segment (start 92.950576 61.252) (end 97.730576 56.472) (width 0.2) (layer "F.Cu") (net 26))
 (segment (start 116.5 60.75) (end 95.292468 60.75) (width 2) (layer "F.Cu") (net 28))
 (segment (start 93.489468 62.553) (end 74.122203 62.553) (width 2) (layer "F.Cu") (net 28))
 (segment (start 73.361203 63.314) (end 71.525892 63.314) (width 2) (layer "F.Cu") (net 28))
 (segment (start 119.5 57.75) (end 116.5 60.75) (width 2) (layer "F.Cu") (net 28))
 (segment (start 142.99 55.51) (end 140.75 57.75) (width 2) (layer "F.Cu") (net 28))
 (segment (start 162.9 55.51) (end 142.99 55.51) (width 2) (layer "F.Cu") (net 28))
 (segment (start 140.75 57.75) (end 119.5 57.75) (width 2) (layer "F.Cu") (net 28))
 (segment (start 68.75 76.522081) (end 66.902081 78.37) (width 2) (layer "F.Cu") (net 28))
 (segment (start 66.902081 78.37) (end 65.7 78.37) (width 2) (layer "F.Cu") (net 28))
 (segment (start 95.292468 60.75) (end 93.489468 62.553) (width 2) (layer "F.Cu") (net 28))
 (segment (start 71.525892 63.314) (end 68.75 66.089892) (width 2) (layer "F.Cu") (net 28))
 (segment (start 74.122203 62.553) (end 73.361203 63.314) (width 2) (layer "F.Cu") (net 28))
 (segment (start 68.75 66.089892) (end 68.75 76.522081) (width 2) (layer "F.Cu") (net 28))
 (segment (start 113.422216 58.112) (end 113.310216 58) (width 2) (layer "F.Cu") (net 6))
 (segment (start 115.839893 58) (end 115.689784 58) (width 2) (layer "F.Cu") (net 6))
 (segment (start 115.577784 58.112) (end 113.422216 58.112) (width 2) (layer "F.Cu") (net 6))
 (segment (start 120.839893 53) (end 115.839893 58) (width 2) (layer "F.Cu") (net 6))
 (segment (start 115.689784 58) (end 115.577784 58.112) (width 2) (layer "F.Cu") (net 6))
 (segment (start 138.67 53) (end 120.839893 53) (width 2) (layer "F.Cu") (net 6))
 (segment (start 138.7 52.97) (end 138.67 53) (width 2) (layer "F.Cu") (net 6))
 (segment (start 113.310216 58) (end 98.75 58) (width 2) (layer "F.Cu") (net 6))
 (via (at 102.75 58.049) (size 1) (drill 0.5) (layers "F.Cu" "B.Cu") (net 6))
 (via (at 98.25 58.049) (size 1) (drill 0.5) (layers "F.Cu" "B.Cu") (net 6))
 (via (at 99.75 58.049) (size 1) (drill 0.5) (layers "F.Cu" "B.Cu") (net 6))
 (via (at 104.25 58.049) (size 1) (drill 0.5) (layers "F.Cu" "B.Cu") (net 6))
 (via (at 101.25 58.049) (size 1) (drill 0.5) (layers "F.Cu" "B.Cu") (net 6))
 (segment (start 99.75 58.049) (end 98.25 58.049) (width 2) (layer "B.Cu") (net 6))
 (segment (start 104 58.049) (end 102.75 58.049) (width 2) (layer "B.Cu") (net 6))
 (segment (start 68.371 64.838892) (end 67.751 65.458892) (width 2) (layer "B.Cu") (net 6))
 (segment (start 101.25 58.049) (end 99.75 58.049) (width 2) (layer "B.Cu") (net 6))
 (segment (start 68.371 60.129) (end 68.371 64.838892) (width 2) (layer "B.Cu") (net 6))
 (segment (start 67.751 66.519553) (end 66.549553 67.721) (width 2) (layer "B.Cu") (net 6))
 (segment (start 102.75 58.049) (end 101.25 58.049) (width 2) (layer "B.Cu") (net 6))
 (segment (start 104.25 58.049) (end 104 58.049) (width 2) (layer "B.Cu") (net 6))
 (segment (start 65.79 68.3) (end 65.7 68.21) (width 2) (layer "B.Cu") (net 6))
 (segment (start 98.25 58.049) (end 70.451 58.049) (width 2) (layer "B.Cu") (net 6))
 (segment (start 70.451 58.049) (end 68.371 60.129) (width 2) (layer "B.Cu") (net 6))
 (segment (start 66.549553 67.721) (end 65.79 67.721) (width 2) (layer "B.Cu") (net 6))
 (segment (start 65.79 67.721) (end 65.79 68.3) (width 2) (layer "B.Cu") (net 6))
 (segment (start 67.751 65.458892) (end 67.751 66.519553) (width 2) (layer "B.Cu") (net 6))
 (segment (start 67.751 72.744921) (end 67.751 74.139553) (width 2) (layer "B.Cu") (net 27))
 (segment (start 162.9 52.97) (end 145.569892 52.97) (width 2) (layer "B.Cu") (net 27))
 (segment (start 65.7 76.190553) (end 65.7 75.83) (width 2) (layer "B.Cu") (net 27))
 (segment (start 72.773 62.451) (end 72.773 67.722921) (width 2) (layer "B.Cu") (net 27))
 (segment (start 72.773 67.722921) (end 67.751 72.744921) (width 2) (layer "B.Cu") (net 27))
 (segment (start 140.789892 57.75) (end 119.75 57.75) (width 2) (layer "B.Cu") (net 27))
 (segment (start 108.612684 60.25) (end 106.411684 62.451) (width 2) (layer "B.Cu") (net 27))
 (segment (start 67.751 74.139553) (end 65.7 76.190553) (width 2) (layer "B.Cu") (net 27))
 (segment (start 106.411684 62.451) (end 72.773 62.451) (width 2) (layer "B.Cu") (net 27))
 (segment (start 117.25 60.25) (end 108.612684 60.25) (width 2) (layer "B.Cu") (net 27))
 (segment (start 145.569892 52.97) (end 140.789892 57.75) (width 2) (layer "B.Cu") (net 27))
 (segment (start 119.75 57.75) (end 117.25 60.25) (width 2) (layer "B.Cu") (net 27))
 (segment (start 67.280684 69.922) (end 66.701684 70.501) (width 2) (layer "B.Cu") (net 7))
 (segment (start 138.7 55.51) (end 117.400553 55.51) (width 2) (layer "B.Cu") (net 7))
 (segment (start 105.5 60.25) (end 71.362684 60.25) (width 2) (layer "B.Cu") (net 7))
 (segment (start 117.400553 55.51) (end 114.910553 58) (width 2) (layer "B.Cu") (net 7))
 (segment (start 107.75 58) (end 105.5 60.25) (width 2) (layer "B.Cu") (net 7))
 (segment (start 114.910553 58) (end 107.75 58) (width 2) (layer "B.Cu") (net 7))
 (segment (start 67.461237 69.922) (end 67.280684 69.922) (width 2) (layer "B.Cu") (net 7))
 (segment (start 65.7 70.501) (end 65.7 70.75) (width 2) (layer "B.Cu") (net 7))
 (segment (start 71.362684 60.25) (end 70.572 61.040684) (width 2) (layer "B.Cu") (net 7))
 (segment (start 70.572 61.040684) (end 70.572 66.811237) (width 2) (layer "B.Cu") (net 7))
 (segment (start 66.701684 70.501) (end 65.7 70.501) (width 2) (layer "B.Cu") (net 7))
 (segment (start 70.572 66.811237) (end 67.461237 69.922) (width 2) (layer "B.Cu") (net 7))
 (segment (start 68.371735 55.509) (end 67.128265 55.509) (width 2) (layer "F.Cu") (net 10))
 (segment (start 66.928265 55.709) (end 66.201108 55.709) (width 2) (layer "F.Cu") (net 10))
 (segment (start 66.050054 55.860054) (end 65.7 55.51) (width 2) (layer "F.Cu") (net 10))
 (segment (start 67.128265 55.509) (end 66.928265 55.709) (width 2) (layer "F.Cu") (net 10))
 (segment (start 68.411735 55.549) (end 68.371735 55.509) (width 2) (layer "F.Cu") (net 10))
 (segment (start 66.201108 55.709) (end 66.050054 55.860054) (width 2) (layer "F.Cu") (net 10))
 (segment (start 90.261 55.549) (end 68.411735 55.549) (width 2) (layer "F.Cu") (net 10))
 (segment (start 90.3 55.51) (end 90.261 55.549) (width 2) (layer "F.Cu") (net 10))
 (segment (start 90.3 50.43) (end 65.7 50.43) (width 0.2) (layer "F.Cu") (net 8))
 (segment (start 66.74 57.01) (end 65.7 58.05) (width 0.2) (layer "F.Cu") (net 15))
 (segment (start 67.75 57.01) (end 66.74 57.01) (width 0.2) (layer "F.Cu") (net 15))
 (via (at 67.75 57.01) (size 0.6) (drill 0.3) (layers "F.Cu" "B.Cu") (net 15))
 (segment (start 67.75 57.01) (end 67.75 57) (width 0.2) (layer "B.Cu") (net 15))
 (segment (start 73.169 51.581) (end 113.349 51.581) (width 0.2) (layer "B.Cu") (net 15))
 (segment (start 67.75 57) (end 73.169 51.581) (width 0.2) (layer "B.Cu") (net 15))
 (segment (start 113.349 51.581) (end 114.5 50.43) (width 0.2) (layer "B.Cu") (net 15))
 (segment (start 66.189 60.101) (end 65.7 60.59) (width 2) (layer "F.Cu") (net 16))
 (segment (start 68.371735 58.511) (end 68.139553 58.511) (width 2) (layer "F.Cu") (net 16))
 (segment (start 66.549553 60.101) (end 66.189 60.101) (width 2) (layer "F.Cu") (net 16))
 (segment (start 69.132735 57.75) (end 68.371735 58.511) (width 2) (layer "F.Cu") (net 16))
 (segment (start 91.5 57.75) (end 69.132735 57.75) (width 2) (layer "F.Cu") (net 16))
 (segment (start 114.5 52.97) (end 96.28 52.97) (width 2) (layer "F.Cu") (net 16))
 (segment (start 68.139553 58.511) (end 66.549553 60.101) (width 2) (layer "F.Cu") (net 16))
 (segment (start 96.28 52.97) (end 91.5 57.75) (width 2) (layer "F.Cu") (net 16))
 (segment (start 90.3 52.97) (end 65.7 52.97) (width 2) (layer "F.Cu") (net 9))
 (segment (start 65.7 63.13) (end 66.633237 63.13) (width 2) (layer "F.Cu") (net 17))
 (segment (start 69.283419 60.712) (end 70.044419 59.951) (width 2) (layer "F.Cu") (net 17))
 (segment (start 114.161 55.171) (end 114.5 55.51) (width 2) (layer "F.Cu") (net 17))
 (segment (start 69.051237 60.712) (end 69.283419 60.712) (width 2) (layer "F.Cu") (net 17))
 (segment (start 97.191684 55.171) (end 114.161 55.171) (width 2) (layer "F.Cu") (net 17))
 (segment (start 70.044419 59.951) (end 92.411684 59.951) (width 2) (layer "F.Cu") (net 17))
 (segment (start 92.411684 59.951) (end 97.191684 55.171) (width 2) (layer "F.Cu") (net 17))
 (segment (start 66.633237 63.13) (end 69.051237 60.712) (width 2) (layer "F.Cu") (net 17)))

